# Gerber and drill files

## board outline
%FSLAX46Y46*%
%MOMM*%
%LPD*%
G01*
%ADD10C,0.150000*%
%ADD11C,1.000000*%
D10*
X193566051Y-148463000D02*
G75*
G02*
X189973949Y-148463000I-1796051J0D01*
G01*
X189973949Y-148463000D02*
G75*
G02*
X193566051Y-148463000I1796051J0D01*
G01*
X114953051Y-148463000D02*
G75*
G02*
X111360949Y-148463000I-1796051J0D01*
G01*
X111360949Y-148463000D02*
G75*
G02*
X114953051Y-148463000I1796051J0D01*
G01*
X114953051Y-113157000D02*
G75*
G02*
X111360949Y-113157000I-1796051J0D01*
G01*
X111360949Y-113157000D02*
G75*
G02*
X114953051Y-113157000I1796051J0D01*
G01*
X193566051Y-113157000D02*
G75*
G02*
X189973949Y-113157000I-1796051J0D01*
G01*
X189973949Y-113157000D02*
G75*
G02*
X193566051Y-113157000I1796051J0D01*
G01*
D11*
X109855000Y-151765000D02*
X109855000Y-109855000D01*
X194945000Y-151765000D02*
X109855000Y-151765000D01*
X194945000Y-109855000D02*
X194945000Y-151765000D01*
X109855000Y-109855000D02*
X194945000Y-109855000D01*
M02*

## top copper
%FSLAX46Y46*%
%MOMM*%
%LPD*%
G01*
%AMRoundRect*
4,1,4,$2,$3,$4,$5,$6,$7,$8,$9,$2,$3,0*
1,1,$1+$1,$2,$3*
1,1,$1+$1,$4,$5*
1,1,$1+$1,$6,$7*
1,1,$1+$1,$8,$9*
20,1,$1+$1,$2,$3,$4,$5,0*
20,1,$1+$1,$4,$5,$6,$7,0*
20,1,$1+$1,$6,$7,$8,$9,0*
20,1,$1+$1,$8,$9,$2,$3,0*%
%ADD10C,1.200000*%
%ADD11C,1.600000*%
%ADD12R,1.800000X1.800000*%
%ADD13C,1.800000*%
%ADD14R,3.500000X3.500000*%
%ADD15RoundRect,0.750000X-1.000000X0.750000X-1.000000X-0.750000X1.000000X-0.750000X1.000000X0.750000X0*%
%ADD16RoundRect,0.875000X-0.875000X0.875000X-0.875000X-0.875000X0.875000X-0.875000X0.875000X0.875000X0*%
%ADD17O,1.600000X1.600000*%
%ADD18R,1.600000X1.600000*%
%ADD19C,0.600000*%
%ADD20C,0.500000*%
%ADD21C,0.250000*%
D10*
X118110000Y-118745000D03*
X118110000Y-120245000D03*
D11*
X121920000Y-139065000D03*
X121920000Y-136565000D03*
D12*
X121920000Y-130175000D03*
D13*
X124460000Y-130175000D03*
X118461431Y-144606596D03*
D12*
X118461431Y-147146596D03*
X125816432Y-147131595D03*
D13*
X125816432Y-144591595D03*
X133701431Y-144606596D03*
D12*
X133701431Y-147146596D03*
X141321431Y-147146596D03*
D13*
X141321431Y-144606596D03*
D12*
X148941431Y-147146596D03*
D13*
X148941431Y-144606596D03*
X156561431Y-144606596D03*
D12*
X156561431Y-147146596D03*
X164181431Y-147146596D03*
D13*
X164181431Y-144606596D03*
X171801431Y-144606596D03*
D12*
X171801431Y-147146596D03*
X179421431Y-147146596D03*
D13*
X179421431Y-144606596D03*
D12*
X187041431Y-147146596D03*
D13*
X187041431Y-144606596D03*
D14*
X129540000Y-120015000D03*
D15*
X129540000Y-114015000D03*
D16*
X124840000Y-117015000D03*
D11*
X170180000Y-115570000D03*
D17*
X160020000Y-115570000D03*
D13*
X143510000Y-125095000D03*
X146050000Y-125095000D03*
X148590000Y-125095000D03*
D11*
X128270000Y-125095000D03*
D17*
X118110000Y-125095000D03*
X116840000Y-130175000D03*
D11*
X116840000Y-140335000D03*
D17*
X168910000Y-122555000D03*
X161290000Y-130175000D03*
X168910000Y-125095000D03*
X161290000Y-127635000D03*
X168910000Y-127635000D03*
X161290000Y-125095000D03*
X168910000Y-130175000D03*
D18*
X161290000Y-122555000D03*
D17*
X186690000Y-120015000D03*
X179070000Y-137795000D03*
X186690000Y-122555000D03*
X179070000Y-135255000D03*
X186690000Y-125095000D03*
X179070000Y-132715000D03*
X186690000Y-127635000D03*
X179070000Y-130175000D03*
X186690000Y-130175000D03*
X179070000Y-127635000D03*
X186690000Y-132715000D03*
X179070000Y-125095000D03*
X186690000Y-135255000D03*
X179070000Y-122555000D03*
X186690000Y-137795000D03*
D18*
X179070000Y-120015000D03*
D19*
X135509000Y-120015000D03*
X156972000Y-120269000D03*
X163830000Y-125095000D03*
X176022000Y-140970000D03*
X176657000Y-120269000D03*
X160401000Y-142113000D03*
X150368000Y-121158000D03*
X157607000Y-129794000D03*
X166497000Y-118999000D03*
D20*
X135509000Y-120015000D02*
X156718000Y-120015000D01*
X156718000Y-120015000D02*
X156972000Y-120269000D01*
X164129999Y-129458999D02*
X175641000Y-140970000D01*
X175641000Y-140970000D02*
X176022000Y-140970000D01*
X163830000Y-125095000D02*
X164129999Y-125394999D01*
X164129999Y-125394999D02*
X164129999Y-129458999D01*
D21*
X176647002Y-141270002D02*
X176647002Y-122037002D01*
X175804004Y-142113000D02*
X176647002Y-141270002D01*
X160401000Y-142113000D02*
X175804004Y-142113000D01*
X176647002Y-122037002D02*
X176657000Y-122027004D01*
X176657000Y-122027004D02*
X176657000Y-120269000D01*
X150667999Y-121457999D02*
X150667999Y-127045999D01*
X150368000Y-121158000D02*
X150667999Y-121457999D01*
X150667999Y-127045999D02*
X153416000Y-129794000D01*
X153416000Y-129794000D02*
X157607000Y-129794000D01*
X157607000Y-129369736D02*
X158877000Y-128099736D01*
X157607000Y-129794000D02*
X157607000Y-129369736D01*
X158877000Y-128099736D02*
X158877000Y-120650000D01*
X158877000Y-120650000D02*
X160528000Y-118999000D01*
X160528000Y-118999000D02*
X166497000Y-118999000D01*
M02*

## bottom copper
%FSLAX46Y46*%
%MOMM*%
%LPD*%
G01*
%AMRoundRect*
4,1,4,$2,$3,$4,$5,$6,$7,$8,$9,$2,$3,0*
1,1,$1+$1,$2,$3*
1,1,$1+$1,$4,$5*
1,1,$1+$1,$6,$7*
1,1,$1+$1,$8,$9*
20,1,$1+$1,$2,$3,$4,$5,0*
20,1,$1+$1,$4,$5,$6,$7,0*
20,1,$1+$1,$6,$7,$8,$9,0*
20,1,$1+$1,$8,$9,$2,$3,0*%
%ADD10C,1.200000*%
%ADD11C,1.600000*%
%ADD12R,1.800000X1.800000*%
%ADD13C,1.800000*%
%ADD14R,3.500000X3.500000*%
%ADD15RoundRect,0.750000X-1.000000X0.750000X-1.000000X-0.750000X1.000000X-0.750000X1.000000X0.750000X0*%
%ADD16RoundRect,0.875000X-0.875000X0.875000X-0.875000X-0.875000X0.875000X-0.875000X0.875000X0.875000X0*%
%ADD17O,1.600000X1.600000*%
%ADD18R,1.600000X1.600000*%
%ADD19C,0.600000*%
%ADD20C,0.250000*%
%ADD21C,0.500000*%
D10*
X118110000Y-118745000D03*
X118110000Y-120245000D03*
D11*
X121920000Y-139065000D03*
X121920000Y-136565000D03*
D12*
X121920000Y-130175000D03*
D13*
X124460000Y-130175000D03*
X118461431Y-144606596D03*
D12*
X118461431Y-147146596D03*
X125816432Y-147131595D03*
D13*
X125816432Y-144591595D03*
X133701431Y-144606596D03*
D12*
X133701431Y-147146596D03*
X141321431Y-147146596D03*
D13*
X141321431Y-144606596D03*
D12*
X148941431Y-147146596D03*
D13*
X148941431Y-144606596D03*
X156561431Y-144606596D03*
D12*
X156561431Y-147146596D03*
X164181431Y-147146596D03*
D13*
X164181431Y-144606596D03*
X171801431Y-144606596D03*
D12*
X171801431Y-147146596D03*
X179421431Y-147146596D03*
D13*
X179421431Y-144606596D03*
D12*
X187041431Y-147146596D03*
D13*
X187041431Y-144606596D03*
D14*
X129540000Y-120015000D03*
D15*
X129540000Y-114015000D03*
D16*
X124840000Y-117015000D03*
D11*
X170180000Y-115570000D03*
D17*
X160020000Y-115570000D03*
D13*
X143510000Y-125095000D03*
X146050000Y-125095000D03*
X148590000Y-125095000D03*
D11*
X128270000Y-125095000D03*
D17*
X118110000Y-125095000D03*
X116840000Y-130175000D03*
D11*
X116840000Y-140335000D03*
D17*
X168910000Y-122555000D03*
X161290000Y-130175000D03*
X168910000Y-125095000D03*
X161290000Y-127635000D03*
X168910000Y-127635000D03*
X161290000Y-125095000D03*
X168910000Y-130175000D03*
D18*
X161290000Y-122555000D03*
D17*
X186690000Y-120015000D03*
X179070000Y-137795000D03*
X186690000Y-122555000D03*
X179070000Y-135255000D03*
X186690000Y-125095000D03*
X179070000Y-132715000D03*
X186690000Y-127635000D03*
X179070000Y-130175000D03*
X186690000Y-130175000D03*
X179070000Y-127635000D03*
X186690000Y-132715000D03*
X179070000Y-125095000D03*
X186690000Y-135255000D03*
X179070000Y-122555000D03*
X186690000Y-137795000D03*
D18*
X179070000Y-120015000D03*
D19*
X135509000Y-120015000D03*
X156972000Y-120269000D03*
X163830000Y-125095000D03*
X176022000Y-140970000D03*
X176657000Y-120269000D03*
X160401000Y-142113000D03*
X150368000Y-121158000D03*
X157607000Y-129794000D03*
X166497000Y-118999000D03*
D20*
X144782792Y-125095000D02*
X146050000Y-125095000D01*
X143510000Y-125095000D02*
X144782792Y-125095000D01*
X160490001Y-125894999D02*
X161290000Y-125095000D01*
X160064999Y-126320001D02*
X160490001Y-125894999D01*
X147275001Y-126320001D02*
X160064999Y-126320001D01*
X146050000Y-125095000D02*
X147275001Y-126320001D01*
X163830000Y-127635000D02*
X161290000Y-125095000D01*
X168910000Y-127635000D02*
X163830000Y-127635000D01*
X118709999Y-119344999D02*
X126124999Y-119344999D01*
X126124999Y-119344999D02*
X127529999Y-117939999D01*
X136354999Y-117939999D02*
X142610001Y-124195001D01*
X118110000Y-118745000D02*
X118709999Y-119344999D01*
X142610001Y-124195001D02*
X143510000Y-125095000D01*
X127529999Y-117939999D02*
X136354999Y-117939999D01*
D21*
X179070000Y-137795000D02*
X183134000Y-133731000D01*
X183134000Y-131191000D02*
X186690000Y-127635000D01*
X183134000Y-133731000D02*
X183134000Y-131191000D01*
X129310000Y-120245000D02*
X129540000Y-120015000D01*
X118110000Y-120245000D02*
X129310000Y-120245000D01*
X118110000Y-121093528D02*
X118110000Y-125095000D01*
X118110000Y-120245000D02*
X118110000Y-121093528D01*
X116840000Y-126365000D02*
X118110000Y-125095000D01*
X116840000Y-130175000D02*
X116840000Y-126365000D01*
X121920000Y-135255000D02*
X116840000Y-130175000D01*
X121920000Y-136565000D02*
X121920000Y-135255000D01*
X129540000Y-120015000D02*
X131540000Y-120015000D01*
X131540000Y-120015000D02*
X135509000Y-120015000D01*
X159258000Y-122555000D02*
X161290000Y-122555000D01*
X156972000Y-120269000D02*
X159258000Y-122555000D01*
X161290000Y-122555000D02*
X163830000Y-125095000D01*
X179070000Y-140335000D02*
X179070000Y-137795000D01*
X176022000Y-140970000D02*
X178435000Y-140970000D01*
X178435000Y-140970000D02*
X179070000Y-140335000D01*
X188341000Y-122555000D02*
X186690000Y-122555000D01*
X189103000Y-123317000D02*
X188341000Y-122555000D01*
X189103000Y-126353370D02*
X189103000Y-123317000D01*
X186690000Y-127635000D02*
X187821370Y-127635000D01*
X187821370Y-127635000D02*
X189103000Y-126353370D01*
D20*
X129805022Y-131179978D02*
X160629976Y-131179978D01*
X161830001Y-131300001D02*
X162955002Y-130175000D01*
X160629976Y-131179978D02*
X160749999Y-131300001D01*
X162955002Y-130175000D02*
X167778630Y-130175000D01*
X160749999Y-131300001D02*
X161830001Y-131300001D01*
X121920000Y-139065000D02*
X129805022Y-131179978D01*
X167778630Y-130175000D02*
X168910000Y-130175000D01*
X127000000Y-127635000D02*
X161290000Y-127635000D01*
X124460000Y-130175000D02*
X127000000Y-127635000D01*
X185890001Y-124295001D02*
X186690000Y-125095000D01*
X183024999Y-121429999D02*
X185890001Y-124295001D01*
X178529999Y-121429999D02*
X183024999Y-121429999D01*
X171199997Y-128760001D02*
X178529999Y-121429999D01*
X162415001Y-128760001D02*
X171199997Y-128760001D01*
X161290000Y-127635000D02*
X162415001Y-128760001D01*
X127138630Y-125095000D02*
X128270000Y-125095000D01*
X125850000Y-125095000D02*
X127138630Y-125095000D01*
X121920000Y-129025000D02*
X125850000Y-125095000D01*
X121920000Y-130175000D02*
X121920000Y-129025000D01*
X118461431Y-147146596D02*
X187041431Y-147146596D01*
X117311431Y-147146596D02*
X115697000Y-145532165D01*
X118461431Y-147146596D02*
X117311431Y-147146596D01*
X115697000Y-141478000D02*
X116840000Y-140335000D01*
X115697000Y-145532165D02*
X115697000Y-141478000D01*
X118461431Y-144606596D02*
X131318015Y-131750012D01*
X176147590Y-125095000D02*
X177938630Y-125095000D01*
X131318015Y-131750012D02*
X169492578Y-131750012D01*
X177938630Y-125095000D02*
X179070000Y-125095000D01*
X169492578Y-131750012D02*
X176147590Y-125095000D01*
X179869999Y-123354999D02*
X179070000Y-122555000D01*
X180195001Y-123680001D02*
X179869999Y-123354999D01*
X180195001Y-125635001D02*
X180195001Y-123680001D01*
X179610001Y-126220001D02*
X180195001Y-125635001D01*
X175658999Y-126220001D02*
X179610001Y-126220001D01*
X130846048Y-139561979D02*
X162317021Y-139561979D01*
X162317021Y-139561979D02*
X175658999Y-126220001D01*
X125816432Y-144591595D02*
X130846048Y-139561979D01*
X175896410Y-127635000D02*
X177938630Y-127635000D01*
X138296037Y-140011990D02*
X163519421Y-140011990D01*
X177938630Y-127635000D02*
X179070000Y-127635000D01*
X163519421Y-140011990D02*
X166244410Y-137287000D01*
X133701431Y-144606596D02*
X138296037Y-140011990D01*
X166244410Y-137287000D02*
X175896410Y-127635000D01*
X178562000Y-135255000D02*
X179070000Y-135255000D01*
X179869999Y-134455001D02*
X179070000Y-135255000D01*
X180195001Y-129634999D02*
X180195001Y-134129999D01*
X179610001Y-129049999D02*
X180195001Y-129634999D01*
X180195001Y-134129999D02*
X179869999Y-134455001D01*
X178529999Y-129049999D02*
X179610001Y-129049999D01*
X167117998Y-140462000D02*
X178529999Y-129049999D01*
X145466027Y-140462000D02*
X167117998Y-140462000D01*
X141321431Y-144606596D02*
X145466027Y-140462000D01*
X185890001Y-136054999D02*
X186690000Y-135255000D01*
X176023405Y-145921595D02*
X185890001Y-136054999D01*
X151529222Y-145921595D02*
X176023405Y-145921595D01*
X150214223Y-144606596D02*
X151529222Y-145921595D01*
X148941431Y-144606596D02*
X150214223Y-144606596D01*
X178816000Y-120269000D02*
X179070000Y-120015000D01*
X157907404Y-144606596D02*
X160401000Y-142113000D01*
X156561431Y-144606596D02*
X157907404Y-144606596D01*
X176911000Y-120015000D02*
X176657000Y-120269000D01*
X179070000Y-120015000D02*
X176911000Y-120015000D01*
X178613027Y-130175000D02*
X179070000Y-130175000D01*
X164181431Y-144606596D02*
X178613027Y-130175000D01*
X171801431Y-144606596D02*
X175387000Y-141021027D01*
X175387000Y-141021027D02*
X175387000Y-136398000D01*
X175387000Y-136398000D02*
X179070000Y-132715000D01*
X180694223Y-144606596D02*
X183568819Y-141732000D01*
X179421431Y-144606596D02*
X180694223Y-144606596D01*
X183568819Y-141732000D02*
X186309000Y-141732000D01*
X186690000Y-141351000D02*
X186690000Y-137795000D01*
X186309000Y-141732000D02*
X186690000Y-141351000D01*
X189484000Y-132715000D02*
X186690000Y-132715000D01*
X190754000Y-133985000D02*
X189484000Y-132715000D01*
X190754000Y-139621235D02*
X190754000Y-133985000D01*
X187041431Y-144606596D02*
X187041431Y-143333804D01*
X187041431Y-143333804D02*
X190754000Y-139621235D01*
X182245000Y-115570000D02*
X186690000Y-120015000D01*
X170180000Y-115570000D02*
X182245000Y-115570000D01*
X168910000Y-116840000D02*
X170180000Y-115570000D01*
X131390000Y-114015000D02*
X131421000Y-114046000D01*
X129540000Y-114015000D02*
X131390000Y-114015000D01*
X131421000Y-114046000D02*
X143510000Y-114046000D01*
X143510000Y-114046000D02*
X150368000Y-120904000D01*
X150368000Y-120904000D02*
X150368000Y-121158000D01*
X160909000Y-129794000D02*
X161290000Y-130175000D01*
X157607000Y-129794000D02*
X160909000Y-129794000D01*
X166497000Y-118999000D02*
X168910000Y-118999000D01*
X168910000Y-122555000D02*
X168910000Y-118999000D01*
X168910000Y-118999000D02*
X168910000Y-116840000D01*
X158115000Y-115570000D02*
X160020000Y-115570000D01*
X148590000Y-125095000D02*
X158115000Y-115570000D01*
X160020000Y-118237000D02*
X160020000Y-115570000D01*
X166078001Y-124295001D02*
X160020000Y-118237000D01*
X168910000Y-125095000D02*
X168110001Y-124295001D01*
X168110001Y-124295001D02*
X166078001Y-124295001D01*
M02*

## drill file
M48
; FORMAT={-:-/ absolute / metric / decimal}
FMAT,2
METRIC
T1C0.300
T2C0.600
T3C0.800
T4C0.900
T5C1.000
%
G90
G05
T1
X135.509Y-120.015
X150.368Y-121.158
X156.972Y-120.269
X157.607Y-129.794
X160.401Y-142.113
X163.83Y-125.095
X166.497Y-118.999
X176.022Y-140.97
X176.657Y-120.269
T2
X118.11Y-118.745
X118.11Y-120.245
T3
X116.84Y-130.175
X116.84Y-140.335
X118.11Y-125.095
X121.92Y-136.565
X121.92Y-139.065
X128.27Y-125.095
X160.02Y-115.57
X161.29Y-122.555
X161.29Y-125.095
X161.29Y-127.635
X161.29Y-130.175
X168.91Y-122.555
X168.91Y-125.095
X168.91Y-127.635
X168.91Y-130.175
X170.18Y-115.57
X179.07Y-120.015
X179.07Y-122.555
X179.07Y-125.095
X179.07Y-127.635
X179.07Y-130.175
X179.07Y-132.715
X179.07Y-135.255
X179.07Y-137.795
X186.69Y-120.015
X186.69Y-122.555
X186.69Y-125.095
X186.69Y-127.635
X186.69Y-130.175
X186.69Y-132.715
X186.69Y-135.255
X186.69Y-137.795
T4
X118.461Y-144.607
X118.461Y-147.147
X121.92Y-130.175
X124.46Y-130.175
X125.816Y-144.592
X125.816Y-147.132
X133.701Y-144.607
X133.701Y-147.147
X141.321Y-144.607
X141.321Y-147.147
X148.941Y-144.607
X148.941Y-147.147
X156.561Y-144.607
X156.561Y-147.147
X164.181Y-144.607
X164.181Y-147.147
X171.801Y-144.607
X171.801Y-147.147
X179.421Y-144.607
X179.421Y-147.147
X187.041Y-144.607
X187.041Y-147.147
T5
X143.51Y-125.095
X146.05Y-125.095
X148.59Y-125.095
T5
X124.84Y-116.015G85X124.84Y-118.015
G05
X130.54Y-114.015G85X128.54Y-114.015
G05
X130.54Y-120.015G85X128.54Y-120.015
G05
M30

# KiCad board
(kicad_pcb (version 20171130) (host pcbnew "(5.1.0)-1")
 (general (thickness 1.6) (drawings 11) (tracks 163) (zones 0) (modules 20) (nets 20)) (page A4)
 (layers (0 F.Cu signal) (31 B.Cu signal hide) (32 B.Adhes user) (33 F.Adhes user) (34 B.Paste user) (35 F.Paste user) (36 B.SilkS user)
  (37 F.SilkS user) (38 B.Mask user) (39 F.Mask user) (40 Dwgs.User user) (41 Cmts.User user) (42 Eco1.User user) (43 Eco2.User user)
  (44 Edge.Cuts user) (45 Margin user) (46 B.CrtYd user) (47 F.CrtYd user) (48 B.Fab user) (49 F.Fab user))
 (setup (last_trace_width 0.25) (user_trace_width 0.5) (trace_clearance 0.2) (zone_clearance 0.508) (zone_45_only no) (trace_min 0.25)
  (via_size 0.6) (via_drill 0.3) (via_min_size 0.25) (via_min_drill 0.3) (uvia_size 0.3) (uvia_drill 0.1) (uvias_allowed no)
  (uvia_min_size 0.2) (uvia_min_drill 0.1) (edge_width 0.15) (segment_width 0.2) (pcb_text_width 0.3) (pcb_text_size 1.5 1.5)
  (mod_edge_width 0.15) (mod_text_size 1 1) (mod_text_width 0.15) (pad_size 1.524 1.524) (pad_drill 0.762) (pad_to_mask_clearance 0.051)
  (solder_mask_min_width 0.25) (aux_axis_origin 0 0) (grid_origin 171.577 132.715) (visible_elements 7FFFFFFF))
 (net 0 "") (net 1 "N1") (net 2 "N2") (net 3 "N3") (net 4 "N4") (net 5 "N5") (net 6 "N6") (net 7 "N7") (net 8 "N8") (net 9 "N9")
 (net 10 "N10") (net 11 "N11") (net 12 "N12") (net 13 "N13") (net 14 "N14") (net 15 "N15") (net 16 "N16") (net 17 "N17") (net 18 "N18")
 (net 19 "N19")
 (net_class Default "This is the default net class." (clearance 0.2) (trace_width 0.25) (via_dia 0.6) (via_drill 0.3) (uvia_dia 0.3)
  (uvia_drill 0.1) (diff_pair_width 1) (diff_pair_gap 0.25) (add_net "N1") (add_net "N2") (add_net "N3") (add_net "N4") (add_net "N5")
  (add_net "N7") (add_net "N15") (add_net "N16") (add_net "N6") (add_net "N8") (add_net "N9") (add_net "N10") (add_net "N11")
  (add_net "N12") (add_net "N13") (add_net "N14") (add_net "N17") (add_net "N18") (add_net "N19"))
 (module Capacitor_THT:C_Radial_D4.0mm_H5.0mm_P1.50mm (layer F.Cu) (at 118.11 118.745 270)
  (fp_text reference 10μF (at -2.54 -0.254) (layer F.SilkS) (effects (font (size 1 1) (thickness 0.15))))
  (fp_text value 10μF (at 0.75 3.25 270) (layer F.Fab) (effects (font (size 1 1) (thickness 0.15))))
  (pad 1 thru_hole circle (at 0 0 270) (size 1.2 1.2) (drill 0.6) (layers *.Cu *.Mask) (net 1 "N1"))
  (pad 2 thru_hole circle (at 1.5 0 270) (size 1.2 1.2) (drill 0.6) (layers *.Cu *.Mask) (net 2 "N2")))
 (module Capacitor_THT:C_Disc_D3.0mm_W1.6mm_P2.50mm (layer F.Cu) (at 121.92 139.065 90)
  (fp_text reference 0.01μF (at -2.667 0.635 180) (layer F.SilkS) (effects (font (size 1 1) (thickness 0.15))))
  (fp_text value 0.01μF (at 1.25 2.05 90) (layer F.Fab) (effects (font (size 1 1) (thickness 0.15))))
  (pad 1 thru_hole circle (at 0 0 90) (size 1.6 1.6) (drill 0.8) (layers *.Cu *.Mask) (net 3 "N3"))
  (pad 2 thru_hole circle (at 2.5 0 90) (size 1.6 1.6) (drill 0.8) (layers *.Cu *.Mask) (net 2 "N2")))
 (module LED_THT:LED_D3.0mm (layer F.Cu) (at 121.92 130.175)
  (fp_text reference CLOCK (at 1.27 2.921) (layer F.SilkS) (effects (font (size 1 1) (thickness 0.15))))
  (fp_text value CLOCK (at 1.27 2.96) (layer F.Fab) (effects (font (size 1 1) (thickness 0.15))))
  (pad 1 thru_hole rect (at 0 0) (size 1.8 1.8) (drill 0.9) (layers *.Cu *.Mask) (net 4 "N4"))
  (pad 2 thru_hole circle (at 2.54 0) (size 1.8 1.8) (drill 0.9) (layers *.Cu *.Mask) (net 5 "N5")))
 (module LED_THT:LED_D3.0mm (layer F.Cu) (at 118.461431 147.146596 90)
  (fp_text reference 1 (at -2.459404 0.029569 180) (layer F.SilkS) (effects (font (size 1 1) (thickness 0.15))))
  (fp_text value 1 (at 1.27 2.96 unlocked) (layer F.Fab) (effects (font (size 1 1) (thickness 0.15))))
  (pad 2 thru_hole circle (at 2.54 0 90) (size 1.8 1.8) (drill 0.9) (layers *.Cu *.Mask) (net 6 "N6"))
  (pad 1 thru_hole rect (at 0 0 90) (size 1.8 1.8) (drill 0.9) (layers *.Cu *.Mask) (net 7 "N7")))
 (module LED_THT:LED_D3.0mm (layer F.Cu) (at 125.816432 147.131595 90)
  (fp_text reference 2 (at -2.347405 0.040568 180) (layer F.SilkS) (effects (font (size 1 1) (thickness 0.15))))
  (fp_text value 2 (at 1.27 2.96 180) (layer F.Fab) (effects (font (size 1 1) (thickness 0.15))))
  (pad 1 thru_hole rect (at 0 0 90) (size 1.8 1.8) (drill 0.9) (layers *.Cu *.Mask) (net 7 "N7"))
  (pad 2 thru_hole circle (at 2.54 0 90) (size 1.8 1.8) (drill 0.9) (layers *.Cu *.Mask) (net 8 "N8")))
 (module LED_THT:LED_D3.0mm (layer F.Cu) (at 133.701431 147.146596 90)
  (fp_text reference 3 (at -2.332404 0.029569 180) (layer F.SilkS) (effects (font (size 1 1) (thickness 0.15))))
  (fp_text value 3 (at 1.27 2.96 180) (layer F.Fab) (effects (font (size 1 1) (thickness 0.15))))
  (pad 2 thru_hole circle (at 2.54 0 90) (size 1.8 1.8) (drill 0.9) (layers *.Cu *.Mask) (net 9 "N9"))
  (pad 1 thru_hole rect (at 0 0 90) (size 1.8 1.8) (drill 0.9) (layers *.Cu *.Mask) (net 7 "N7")))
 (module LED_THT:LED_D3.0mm (layer F.Cu) (at 141.321431 147.146596 90)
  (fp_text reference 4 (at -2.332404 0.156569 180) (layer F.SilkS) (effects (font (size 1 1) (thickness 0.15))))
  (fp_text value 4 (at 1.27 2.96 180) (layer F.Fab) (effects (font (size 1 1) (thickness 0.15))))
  (pad 1 thru_hole rect (at 0 0 90) (size 1.8 1.8) (drill 0.9) (layers *.Cu *.Mask) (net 7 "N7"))
  (pad 2 thru_hole circle (at 2.54 0 90) (size 1.8 1.8) (drill 0.9) (layers *.Cu *.Mask) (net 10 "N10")))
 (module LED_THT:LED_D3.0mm (layer F.Cu) (at 148.941431 147.146596 90)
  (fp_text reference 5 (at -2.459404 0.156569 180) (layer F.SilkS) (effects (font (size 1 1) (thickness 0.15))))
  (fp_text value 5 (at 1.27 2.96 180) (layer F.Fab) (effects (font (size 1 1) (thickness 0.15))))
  (pad 1 thru_hole rect (at 0 0 90) (size 1.8 1.8) (drill 0.9) (layers *.Cu *.Mask) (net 7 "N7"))
  (pad 2 thru_hole circle (at 2.54 0 90) (size 1.8 1.8) (drill 0.9) (layers *.Cu *.Mask) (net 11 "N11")))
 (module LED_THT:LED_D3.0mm (layer F.Cu) (at 156.561431 147.146596 90)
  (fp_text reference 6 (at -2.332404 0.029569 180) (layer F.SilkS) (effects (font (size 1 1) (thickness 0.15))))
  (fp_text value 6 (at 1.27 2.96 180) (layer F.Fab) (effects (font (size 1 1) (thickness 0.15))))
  (pad 2 thru_hole circle (at 2.54 0 90) (size 1.8 1.8) (drill 0.9) (layers *.Cu *.Mask) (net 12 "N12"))
  (pad 1 thru_hole rect (at 0 0 90) (size 1.8 1.8) (drill 0.9) (layers *.Cu *.Mask) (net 7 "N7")))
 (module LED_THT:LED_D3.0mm (layer F.Cu) (at 164.181431 147.146596 90)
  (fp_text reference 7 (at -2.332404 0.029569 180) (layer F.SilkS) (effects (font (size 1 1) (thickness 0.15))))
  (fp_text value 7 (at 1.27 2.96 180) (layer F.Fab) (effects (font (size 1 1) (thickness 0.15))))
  (pad 1 thru_hole rect (at 0 0 90) (size 1.8 1.8) (drill 0.9) (layers *.Cu *.Mask) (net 7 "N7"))
  (pad 2 thru_hole circle (at 2.54 0 90) (size 1.8 1.8) (drill 0.9) (layers *.Cu *.Mask) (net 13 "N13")))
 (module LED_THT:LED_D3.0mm (layer F.Cu) (at 171.801431 147.146596 90)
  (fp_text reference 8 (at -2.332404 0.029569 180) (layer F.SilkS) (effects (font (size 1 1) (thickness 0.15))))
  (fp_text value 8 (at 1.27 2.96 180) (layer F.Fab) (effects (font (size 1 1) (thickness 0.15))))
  (pad 2 thru_hole circle (at 2.54 0 90) (size 1.8 1.8) (drill 0.9) (layers *.Cu *.Mask) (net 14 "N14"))
  (pad 1 thru_hole rect (at 0 0 90) (size 1.8 1.8) (drill 0.9) (layers *.Cu *.Mask) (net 7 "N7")))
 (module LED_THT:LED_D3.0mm (layer F.Cu) (at 179.421431 147.146596 90)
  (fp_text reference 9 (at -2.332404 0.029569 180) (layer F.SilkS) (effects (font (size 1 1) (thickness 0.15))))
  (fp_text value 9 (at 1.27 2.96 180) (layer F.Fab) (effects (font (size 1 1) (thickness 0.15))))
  (pad 1 thru_hole rect (at 0 0 90) (size 1.8 1.8) (drill 0.9) (layers *.Cu *.Mask) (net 7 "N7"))
  (pad 2 thru_hole circle (at 2.54 0 90) (size 1.8 1.8) (drill 0.9) (layers *.Cu *.Mask) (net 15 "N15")))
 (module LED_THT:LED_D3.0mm (layer F.Cu) (at 187.041431 147.146596 90)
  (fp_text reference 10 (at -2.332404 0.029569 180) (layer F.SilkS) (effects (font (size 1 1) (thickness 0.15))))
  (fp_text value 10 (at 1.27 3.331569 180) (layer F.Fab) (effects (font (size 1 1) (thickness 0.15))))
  (pad 1 thru_hole rect (at 0 0 90) (size 1.8 1.8) (drill 0.9) (layers *.Cu *.Mask) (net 7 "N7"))
  (pad 2 thru_hole circle (at 2.54 0 90) (size 1.8 1.8) (drill 0.9) (layers *.Cu *.Mask) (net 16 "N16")))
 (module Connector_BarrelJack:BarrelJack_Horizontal (layer F.Cu) (at 129.54 120.015 270)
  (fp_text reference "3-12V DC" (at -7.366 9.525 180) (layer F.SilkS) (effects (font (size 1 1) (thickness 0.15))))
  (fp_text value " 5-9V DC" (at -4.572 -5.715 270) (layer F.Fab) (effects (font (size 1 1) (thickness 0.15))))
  (pad 1 thru_hole rect (at 0 0 270) (size 3.5 3.5) (drill oval 1 3) (layers *.Cu *.Mask) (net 2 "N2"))
  (pad 2 thru_hole roundrect (at -6 0 270) (size 3 3.5) (drill oval 1 3) (layers *.Cu *.Mask) (roundrect_rratio 0.25) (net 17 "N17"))
  (pad 3 thru_hole roundrect (at -3 4.7 270) (size 3.5 3.5) (drill oval 3 1) (layers *.Cu *.Mask) (roundrect_rratio 0.25)))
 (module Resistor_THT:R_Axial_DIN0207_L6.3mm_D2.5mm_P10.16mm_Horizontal (layer F.Cu) (at 170.18 115.57 180)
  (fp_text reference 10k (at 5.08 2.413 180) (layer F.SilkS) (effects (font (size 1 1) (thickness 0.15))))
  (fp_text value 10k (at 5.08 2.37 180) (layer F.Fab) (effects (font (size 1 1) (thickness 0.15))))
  (pad 1 thru_hole circle (at 0 0 180) (size 1.6 1.6) (drill 0.8) (layers *.Cu *.Mask) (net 17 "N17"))
  (pad 2 thru_hole oval (at 10.16 0 180) (size 1.6 1.6) (drill 0.8) (layers *.Cu *.Mask) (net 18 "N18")))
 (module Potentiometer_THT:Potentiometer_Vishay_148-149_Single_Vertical (layer F.Cu) (at 148.59 125.095 90)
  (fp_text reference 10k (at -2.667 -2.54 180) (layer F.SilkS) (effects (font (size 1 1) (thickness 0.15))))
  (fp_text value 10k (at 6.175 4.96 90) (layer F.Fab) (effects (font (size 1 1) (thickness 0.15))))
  (pad 3 thru_hole circle (at 0 -5.08 90) (size 1.8 1.8) (drill 1) (layers *.Cu *.Mask) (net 1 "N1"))
  (pad 2 thru_hole circle (at 0 -2.54 90) (size 1.8 1.8) (drill 1) (layers *.Cu *.Mask) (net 1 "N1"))
  (pad 1 thru_hole circle (at 0 0 90) (size 1.8 1.8) (drill 1) (layers *.Cu *.Mask) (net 18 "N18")))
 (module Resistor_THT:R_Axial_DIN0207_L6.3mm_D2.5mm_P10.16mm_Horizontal (layer F.Cu) (at 128.27 125.095 180)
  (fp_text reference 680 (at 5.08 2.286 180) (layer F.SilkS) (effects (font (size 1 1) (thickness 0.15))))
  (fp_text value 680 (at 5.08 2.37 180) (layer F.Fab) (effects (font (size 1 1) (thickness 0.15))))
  (pad 1 thru_hole circle (at 0 0 180) (size 1.6 1.6) (drill 0.8) (layers *.Cu *.Mask) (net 4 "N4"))
  (pad 2 thru_hole oval (at 10.16 0 180) (size 1.6 1.6) (drill 0.8) (layers *.Cu *.Mask) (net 2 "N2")))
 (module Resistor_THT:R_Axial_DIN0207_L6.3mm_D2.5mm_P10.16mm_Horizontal (layer F.Cu) (at 116.84 140.335 90)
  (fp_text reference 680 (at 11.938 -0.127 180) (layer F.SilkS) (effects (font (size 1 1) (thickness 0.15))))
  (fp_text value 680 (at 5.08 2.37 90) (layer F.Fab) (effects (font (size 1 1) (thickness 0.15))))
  (pad 2 thru_hole oval (at 10.16 0 90) (size 1.6 1.6) (drill 0.8) (layers *.Cu *.Mask) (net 2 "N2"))
  (pad 1 thru_hole circle (at 0 0 90) (size 1.6 1.6) (drill 0.8) (layers *.Cu *.Mask) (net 7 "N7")))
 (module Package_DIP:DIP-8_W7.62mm (layer F.Cu) (at 161.29 122.555)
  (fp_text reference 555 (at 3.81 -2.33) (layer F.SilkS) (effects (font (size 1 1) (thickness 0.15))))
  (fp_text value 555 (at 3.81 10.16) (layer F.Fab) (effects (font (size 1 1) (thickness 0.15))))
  (pad 8 thru_hole oval (at 7.62 0) (size 1.6 1.6) (drill 0.8) (layers *.Cu *.Mask) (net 17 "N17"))
  (pad 4 thru_hole oval (at 0 7.62) (size 1.6 1.6) (drill 0.8) (layers *.Cu *.Mask) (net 17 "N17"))
  (pad 7 thru_hole oval (at 7.62 2.54) (size 1.6 1.6) (drill 0.8) (layers *.Cu *.Mask) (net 18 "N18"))
  (pad 3 thru_hole oval (at 0 5.08) (size 1.6 1.6) (drill 0.8) (layers *.Cu *.Mask) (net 5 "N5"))
  (pad 6 thru_hole oval (at 7.62 5.08) (size 1.6 1.6) (drill 0.8) (layers *.Cu *.Mask) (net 1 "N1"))
  (pad 2 thru_hole oval (at 0 2.54) (size 1.6 1.6) (drill 0.8) (layers *.Cu *.Mask) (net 1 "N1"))
  (pad 5 thru_hole oval (at 7.62 7.62) (size 1.6 1.6) (drill 0.8) (layers *.Cu *.Mask) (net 3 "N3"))
  (pad 1 thru_hole rect (at 0 0) (size 1.6 1.6) (drill 0.8) (layers *.Cu *.Mask) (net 2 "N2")))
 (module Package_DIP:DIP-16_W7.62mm (layer F.Cu) (at 179.07 120.015)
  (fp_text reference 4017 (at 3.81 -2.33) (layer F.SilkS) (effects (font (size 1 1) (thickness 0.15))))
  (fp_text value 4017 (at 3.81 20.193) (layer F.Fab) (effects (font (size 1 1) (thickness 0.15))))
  (pad 16 thru_hole oval (at 7.62 0) (size 1.6 1.6) (drill 0.8) (layers *.Cu *.Mask) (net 17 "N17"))
  (pad 8 thru_hole oval (at 0 17.78) (size 1.6 1.6) (drill 0.8) (layers *.Cu *.Mask) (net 2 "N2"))
  (pad 15 thru_hole oval (at 7.62 2.54) (size 1.6 1.6) (drill 0.8) (layers *.Cu *.Mask) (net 2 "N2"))
  (pad 7 thru_hole oval (at 0 15.24) (size 1.6 1.6) (drill 0.8) (layers *.Cu *.Mask) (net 10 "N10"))
  (pad 14 thru_hole oval (at 7.62 5.08) (size 1.6 1.6) (drill 0.8) (layers *.Cu *.Mask) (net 5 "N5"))
  (pad 6 thru_hole oval (at 0 12.7) (size 1.6 1.6) (drill 0.8) (layers *.Cu *.Mask) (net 14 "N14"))
  (pad 13 thru_hole oval (at 7.62 7.62) (size 1.6 1.6) (drill 0.8) (layers *.Cu *.Mask) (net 2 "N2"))
  (pad 5 thru_hole oval (at 0 10.16) (size 1.6 1.6) (drill 0.8) (layers *.Cu *.Mask) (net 13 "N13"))
  (pad 12 thru_hole oval (at 7.62 10.16) (size 1.6 1.6) (drill 0.8) (layers *.Cu *.Mask) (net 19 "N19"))
  (pad 4 thru_hole oval (at 0 7.62) (size 1.6 1.6) (drill 0.8) (layers *.Cu *.Mask) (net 9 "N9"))
  (pad 11 thru_hole oval (at 7.62 12.7) (size 1.6 1.6) (drill 0.8) (layers *.Cu *.Mask) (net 16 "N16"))
  (pad 3 thru_hole oval (at 0 5.08) (size 1.6 1.6) (drill 0.8) (layers *.Cu *.Mask) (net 6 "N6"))
  (pad 10 thru_hole oval (at 7.62 15.24) (size 1.6 1.6) (drill 0.8) (layers *.Cu *.Mask) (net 11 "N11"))
  (pad 2 thru_hole oval (at 0 2.54) (size 1.6 1.6) (drill 0.8) (layers *.Cu *.Mask) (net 8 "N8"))
  (pad 9 thru_hole oval (at 7.62 17.78) (size 1.6 1.6) (drill 0.8) (layers *.Cu *.Mask) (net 15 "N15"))
  (pad 1 thru_hole rect (at 0 0) (size 1.6 1.6) (drill 0.8) (layers *.Cu *.Mask) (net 12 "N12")))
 (gr_circle (center 191.77 148.463) (end 193.566051 148.463) (layer Edge.Cuts) (width 0.15))
 (gr_circle (center 113.157 148.463) (end 114.953051 148.463) (layer Edge.Cuts) (width 0.15))
 (gr_circle (center 113.157 113.157) (end 114.953051 113.157) (layer Edge.Cuts) (width 0.15))
 (gr_circle (center 191.77 113.157) (end 193.566051 113.157) (layer Edge.Cuts) (width 0.15))
 (gr_line (start 109.855 151.765) (end 109.855 109.855) (layer Edge.Cuts) (width 1))
 (gr_line (start 194.945 151.765) (end 109.855 151.765) (layer Edge.Cuts) (width 1))
 (gr_line (start 194.945 109.855) (end 194.945 151.765) (layer Edge.Cuts) (width 1))
 (gr_line (start 109.855 109.855) (end 194.945 109.855) (layer Edge.Cuts) (width 1))
 (segment (start 144.782792 125.095) (end 146.05 125.095) (width 0.25) (layer B.Cu) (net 1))
 (segment (start 143.51 125.095) (end 144.782792 125.095) (width 0.25) (layer B.Cu) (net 1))
 (segment (start 160.490001 125.894999) (end 161.29 125.095) (width 0.25) (layer B.Cu) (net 1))
 (segment (start 160.064999 126.320001) (end 160.490001 125.894999) (width 0.25) (layer B.Cu) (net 1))
 (segment (start 147.275001 126.320001) (end 160.064999 126.320001) (width 0.25) (layer B.Cu) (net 1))
 (segment (start 146.05 125.095) (end 147.275001 126.320001) (width 0.25) (layer B.Cu) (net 1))
 (segment (start 163.83 127.635) (end 161.29 125.095) (width 0.25) (layer B.Cu) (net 1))
 (segment (start 168.91 127.635) (end 163.83 127.635) (width 0.25) (layer B.Cu) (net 1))
 (segment (start 118.709999 119.344999) (end 126.124999 119.344999) (width 0.25) (layer B.Cu) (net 1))
 (segment (start 126.124999 119.344999) (end 127.529999 117.939999) (width 0.25) (layer B.Cu) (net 1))
 (segment (start 136.354999 117.939999) (end 142.610001 124.195001) (width 0.25) (layer B.Cu) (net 1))
 (segment (start 118.11 118.745) (end 118.709999 119.344999) (width 0.25) (layer B.Cu) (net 1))
 (segment (start 142.610001 124.195001) (end 143.51 125.095) (width 0.25) (layer B.Cu) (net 1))
 (segment (start 127.529999 117.939999) (end 136.354999 117.939999) (width 0.25) (layer B.Cu) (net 1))
 (segment (start 179.07 137.795) (end 183.134 133.731) (width 0.5) (layer B.Cu) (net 2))
 (segment (start 183.134 131.191) (end 186.69 127.635) (width 0.5) (layer B.Cu) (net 2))
 (segment (start 183.134 133.731) (end 183.134 131.191) (width 0.5) (layer B.Cu) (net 2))
 (segment (start 129.31 120.245) (end 129.54 120.015) (width 0.5) (layer B.Cu) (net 2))
 (segment (start 118.11 120.245) (end 129.31 120.245) (width 0.5) (layer B.Cu) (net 2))
 (segment (start 118.11 121.093528) (end 118.11 125.095) (width 0.5) (layer B.Cu) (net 2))
 (segment (start 118.11 120.245) (end 118.11 121.093528) (width 0.5) (layer B.Cu) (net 2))
 (segment (start 116.84 126.365) (end 118.11 125.095) (width 0.5) (layer B.Cu) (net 2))
 (segment (start 116.84 130.175) (end 116.84 126.365) (width 0.5) (layer B.Cu) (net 2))
 (segment (start 121.92 135.255) (end 116.84 130.175) (width 0.5) (layer B.Cu) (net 2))
 (segment (start 121.92 136.565) (end 121.92 135.255) (width 0.5) (layer B.Cu) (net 2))
 (segment (start 129.54 120.015) (end 131.54 120.015) (width 0.5) (layer B.Cu) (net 2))
 (via (at 135.509 120.015) (size 0.6) (drill 0.3) (layers F.Cu B.Cu) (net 2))
 (segment (start 131.54 120.015) (end 135.509 120.015) (width 0.5) (layer B.Cu) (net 2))
 (via (at 156.972 120.269) (size 0.6) (drill 0.3) (layers F.Cu B.Cu) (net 2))
 (segment (start 135.509 120.015) (end 156.718 120.015) (width 0.5) (layer F.Cu) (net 2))
 (segment (start 156.718 120.015) (end 156.972 120.269) (width 0.5) (layer F.Cu) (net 2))
 (segment (start 159.258 122.555) (end 161.29 122.555) (width 0.5) (layer B.Cu) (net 2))
 (segment (start 156.972 120.269) (end 159.258 122.555) (width 0.5) (layer B.Cu) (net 2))
 (via (at 163.83 125.095) (size 0.6) (drill 0.3) (layers F.Cu B.Cu) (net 2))
 (segment (start 164.129999 129.458999) (end 175.641 140.97) (width 0.5) (layer F.Cu) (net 2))
 (segment (start 175.641 140.97) (end 176.022 140.97) (width 0.5) (layer F.Cu) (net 2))
 (via (at 176.022 140.97) (size 0.6) (drill 0.3) (layers F.Cu B.Cu) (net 2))
 (segment (start 163.83 125.095) (end 164.129999 125.394999) (width 0.5) (layer F.Cu) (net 2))
 (segment (start 164.129999 125.394999) (end 164.129999 129.458999) (width 0.5) (layer F.Cu) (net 2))
 (segment (start 161.29 122.555) (end 163.83 125.095) (width 0.5) (layer B.Cu) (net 2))
 (segment (start 179.07 140.335) (end 179.07 137.795) (width 0.5) (layer B.Cu) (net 2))
 (segment (start 176.022 140.97) (end 178.435 140.97) (width 0.5) (layer B.Cu) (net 2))
 (segment (start 178.435 140.97) (end 179.07 140.335) (width 0.5) (layer B.Cu) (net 2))
 (segment (start 188.341 122.555) (end 186.69 122.555) (width 0.5) (layer B.Cu) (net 2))
 (segment (start 189.103 123.317) (end 188.341 122.555) (width 0.5) (layer B.Cu) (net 2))
 (segment (start 189.103 126.35337) (end 189.103 123.317) (width 0.5) (layer B.Cu) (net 2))
 (segment (start 186.69 127.635) (end 187.82137 127.635) (width 0.5) (layer B.Cu) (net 2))
 (segment (start 187.82137 127.635) (end 189.103 126.35337) (width 0.5) (layer B.Cu) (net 2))
 (segment (start 129.805022 131.179978) (end 160.629976 131.179978) (width 0.25) (layer B.Cu) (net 3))
 (segment (start 161.830001 131.300001) (end 162.955002 130.175) (width 0.25) (layer B.Cu) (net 3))
 (segment (start 160.629976 131.179978) (end 160.749999 131.300001) (width 0.25) (layer B.Cu) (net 3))
 (segment (start 162.955002 130.175) (end 167.77863 130.175) (width 0.25) (layer B.Cu) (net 3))
 (segment (start 160.749999 131.300001) (end 161.830001 131.300001) (width 0.25) (layer B.Cu) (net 3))
 (segment (start 121.92 139.065) (end 129.805022 131.179978) (width 0.25) (layer B.Cu) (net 3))
 (segment (start 167.77863 130.175) (end 168.91 130.175) (width 0.25) (layer B.Cu) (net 3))
 (segment (start 127 127.635) (end 161.29 127.635) (width 0.25) (layer B.Cu) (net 5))
 (segment (start 124.46 130.175) (end 127 127.635) (width 0.25) (layer B.Cu) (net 5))
 (segment (start 185.890001 124.295001) (end 186.69 125.095) (width 0.25) (layer B.Cu) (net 5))
 (segment (start 183.024999 121.429999) (end 185.890001 124.295001) (width 0.25) (layer B.Cu) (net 5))
 (segment (start 178.529999 121.429999) (end 183.024999 121.429999) (width 0.25) (layer B.Cu) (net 5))
 (segment (start 171.199997 128.760001) (end 178.529999 121.429999) (width 0.25) (layer B.Cu) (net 5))
 (segment (start 162.415001 128.760001) (end 171.199997 128.760001) (width 0.25) (layer B.Cu) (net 5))
 (segment (start 161.29 127.635) (end 162.415001 128.760001) (width 0.25) (layer B.Cu) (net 5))
 (segment (start 127.13863 125.095) (end 128.27 125.095) (width 0.25) (layer B.Cu) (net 4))
 (segment (start 125.85 125.095) (end 127.13863 125.095) (width 0.25) (layer B.Cu) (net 4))
 (segment (start 121.92 129.025) (end 125.85 125.095) (width 0.25) (layer B.Cu) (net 4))
 (segment (start 121.92 130.175) (end 121.92 129.025) (width 0.25) (layer B.Cu) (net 4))
 (segment (start 118.461431 147.146596) (end 187.041431 147.146596) (width 0.25) (layer B.Cu) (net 7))
 (segment (start 117.311431 147.146596) (end 115.697 145.532165) (width 0.25) (layer B.Cu) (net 7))
 (segment (start 118.461431 147.146596) (end 117.311431 147.146596) (width 0.25) (layer B.Cu) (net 7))
 (segment (start 115.697 141.478) (end 116.84 140.335) (width 0.25) (layer B.Cu) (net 7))
 (segment (start 115.697 145.532165) (end 115.697 141.478) (width 0.25) (layer B.Cu) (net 7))
 (segment (start 118.461431 144.606596) (end 131.318015 131.750012) (width 0.25) (layer B.Cu) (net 6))
 (segment (start 176.14759 125.095) (end 177.93863 125.095) (width 0.25) (layer B.Cu) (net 6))
 (segment (start 131.318015 131.750012) (end 169.492578 131.750012) (width 0.25) (layer B.Cu) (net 6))
 (segment (start 177.93863 125.095) (end 179.07 125.095) (width 0.25) (layer B.Cu) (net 6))
 (segment (start 169.492578 131.750012) (end 176.14759 125.095) (width 0.25) (layer B.Cu) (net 6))
 (segment (start 179.869999 123.354999) (end 179.07 122.555) (width 0.25) (layer B.Cu) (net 8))
 (segment (start 180.195001 123.680001) (end 179.869999 123.354999) (width 0.25) (layer B.Cu) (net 8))
 (segment (start 180.195001 125.635001) (end 180.195001 123.680001) (width 0.25) (layer B.Cu) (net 8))
 (segment (start 179.610001 126.220001) (end 180.195001 125.635001) (width 0.25) (layer B.Cu) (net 8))
 (segment (start 175.658999 126.220001) (end 179.610001 126.220001) (width 0.25) (layer B.Cu) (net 8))
 (segment (start 130.846048 139.561979) (end 162.317021 139.561979) (width 0.25) (layer B.Cu) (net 8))
 (segment (start 162.317021 139.561979) (end 175.658999 126.220001) (width 0.25) (layer B.Cu) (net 8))
 (segment (start 125.816432 144.591595) (end 130.846048 139.561979) (width 0.25) (layer B.Cu) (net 8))
 (segment (start 175.89641 127.635) (end 177.93863 127.635) (width 0.25) (layer B.Cu) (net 9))
 (segment (start 138.296037 140.01199) (end 163.519421 140.01199) (width 0.25) (layer B.Cu) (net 9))
 (segment (start 177.93863 127.635) (end 179.07 127.635) (width 0.25) (layer B.Cu) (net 9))
 (segment (start 163.519421 140.01199) (end 166.24441 137.287) (width 0.25) (layer B.Cu) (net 9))
 (segment (start 133.701431 144.606596) (end 138.296037 140.01199) (width 0.25) (layer B.Cu) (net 9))
 (segment (start 166.24441 137.287) (end 175.89641 127.635) (width 0.25) (layer B.Cu) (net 9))
 (segment (start 178.562 135.255) (end 179.07 135.255) (width 0.25) (layer B.Cu) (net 10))
 (segment (start 179.869999 134.455001) (end 179.07 135.255) (width 0.25) (layer B.Cu) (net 10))
 (segment (start 180.195001 129.634999) (end 180.195001 134.129999) (width 0.25) (layer B.Cu) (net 10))
 (segment (start 179.610001 129.049999) (end 180.195001 129.634999) (width 0.25) (layer B.Cu) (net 10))
 (segment (start 180.195001 134.129999) (end 179.869999 134.455001) (width 0.25) (layer B.Cu) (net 10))
 (segment (start 178.529999 129.049999) (end 179.610001 129.049999) (width 0.25) (layer B.Cu) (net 10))
 (segment (start 167.117998 140.462) (end 178.529999 129.049999) (width 0.25) (layer B.Cu) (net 10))
 (segment (start 145.466027 140.462) (end 167.117998 140.462) (width 0.25) (layer B.Cu) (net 10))
 (segment (start 141.321431 144.606596) (end 145.466027 140.462) (width 0.25) (layer B.Cu) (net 10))
 (segment (start 185.890001 136.054999) (end 186.69 135.255) (width 0.25) (layer B.Cu) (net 11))
 (segment (start 176.023405 145.921595) (end 185.890001 136.054999) (width 0.25) (layer B.Cu) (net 11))
 (segment (start 151.529222 145.921595) (end 176.023405 145.921595) (width 0.25) (layer B.Cu) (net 11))
 (segment (start 150.214223 144.606596) (end 151.529222 145.921595) (width 0.25) (layer B.Cu) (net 11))
 (segment (start 148.941431 144.606596) (end 150.214223 144.606596) (width 0.25) (layer B.Cu) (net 11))
 (segment (start 178.816 120.269) (end 179.07 120.015) (width 0.25) (layer B.Cu) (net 12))
 (segment (start 176.647002 141.270002) (end 176.647002 122.037002) (width 0.25) (layer F.Cu) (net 12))
 (segment (start 175.804004 142.113) (end 176.647002 141.270002) (width 0.25) (layer F.Cu) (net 12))
 (segment (start 160.401 142.113) (end 175.804004 142.113) (width 0.25) (layer F.Cu) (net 12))
 (segment (start 176.647002 122.037002) (end 176.657 122.027004) (width 0.25) (layer F.Cu) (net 12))
 (segment (start 176.657 122.027004) (end 176.657 120.269) (width 0.25) (layer F.Cu) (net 12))
 (via (at 176.657 120.269) (size 0.6) (drill 0.3) (layers F.Cu B.Cu) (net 12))
 (via (at 160.401 142.113) (size 0.6) (drill 0.3) (layers F.Cu B.Cu) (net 12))
 (segment (start 157.907404 144.606596) (end 160.401 142.113) (width 0.25) (layer B.Cu) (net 12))
 (segment (start 156.561431 144.606596) (end 157.907404 144.606596) (width 0.25) (layer B.Cu) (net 12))
 (segment (start 176.911 120.015) (end 176.657 120.269) (width 0.25) (layer B.Cu) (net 12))
 (segment (start 179.07 120.015) (end 176.911 120.015) (width 0.25) (layer B.Cu) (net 12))
 (segment (start 178.613027 130.175) (end 179.07 130.175) (width 0.25) (layer B.Cu) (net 13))
 (segment (start 164.181431 144.606596) (end 178.613027 130.175) (width 0.25) (layer B.Cu) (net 13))
 (segment (start 171.801431 144.606596) (end 175.387 141.021027) (width 0.25) (layer B.Cu) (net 14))
 (segment (start 175.387 141.021027) (end 175.387 136.398) (width 0.25) (layer B.Cu) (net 14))
 (segment (start 175.387 136.398) (end 179.07 132.715) (width 0.25) (layer B.Cu) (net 14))
 (segment (start 180.694223 144.606596) (end 183.568819 141.732) (width 0.25) (layer B.Cu) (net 15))
 (segment (start 179.421431 144.606596) (end 180.694223 144.606596) (width 0.25) (layer B.Cu) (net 15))
 (segment (start 183.568819 141.732) (end 186.309 141.732) (width 0.25) (layer B.Cu) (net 15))
 (segment (start 186.69 141.351) (end 186.69 137.795) (width 0.25) (layer B.Cu) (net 15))
 (segment (start 186.309 141.732) (end 186.69 141.351) (width 0.25) (layer B.Cu) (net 15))
 (segment (start 189.484 132.715) (end 186.69 132.715) (width 0.25) (layer B.Cu) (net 16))
 (segment (start 190.754 133.985) (end 189.484 132.715) (width 0.25) (layer B.Cu) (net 16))
 (segment (start 190.754 139.621235) (end 190.754 133.985) (width 0.25) (layer B.Cu) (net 16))
 (segment (start 187.041431 144.606596) (end 187.041431 143.333804) (width 0.25) (layer B.Cu) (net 16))
 (segment (start 187.041431 143.333804) (end 190.754 139.621235) (width 0.25) (layer B.Cu) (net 16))
 (segment (start 182.245 115.57) (end 186.69 120.015) (width 0.25) (layer B.Cu) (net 17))
 (segment (start 170.18 115.57) (end 182.245 115.57) (width 0.25) (layer B.Cu) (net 17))
 (segment (start 168.91 116.84) (end 170.18 115.57) (width 0.25) (layer B.Cu) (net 17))
 (segment (start 131.39 114.015) (end 131.421 114.046) (width 0.25) (layer B.Cu) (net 17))
 (segment (start 129.54 114.015) (end 131.39 114.015) (width 0.25) (layer B.Cu) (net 17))
 (segment (start 131.421 114.046) (end 143.51 114.046) (width 0.25) (layer B.Cu) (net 17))
 (via (at 150.368 121.158) (size 0.6) (drill 0.3) (layers F.Cu B.Cu) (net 17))
 (segment (start 143.51 114.046) (end 150.368 120.904) (width 0.25) (layer B.Cu) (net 17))
 (segment (start 150.368 120.904) (end 150.368 121.158) (width 0.25) (layer B.Cu) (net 17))
 (segment (start 150.667999 121.457999) (end 150.667999 127.045999) (width 0.25) (layer F.Cu) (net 17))
 (segment (start 150.368 121.158) (end 150.667999 121.457999) (width 0.25) (layer F.Cu) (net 17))
 (segment (start 150.667999 127.045999) (end 153.416 129.794) (width 0.25) (layer F.Cu) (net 17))
 (via (at 157.607 129.794) (size 0.6) (drill 0.3) (layers F.Cu B.Cu) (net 17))
 (segment (start 153.416 129.794) (end 157.607 129.794) (width 0.25) (layer F.Cu) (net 17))
 (segment (start 160.909 129.794) (end 161.29 130.175) (width 0.25) (layer B.Cu) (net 17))
 (segment (start 157.607 129.794) (end 160.909 129.794) (width 0.25) (layer B.Cu) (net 17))
 (segment (start 157.607 129.369736) (end 158.877 128.099736) (width 0.25) (layer F.Cu) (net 17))
 (segment (start 157.607 129.794) (end 157.607 129.369736) (width 0.25) (layer F.Cu) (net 17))
 (segment (start 158.877 128.099736) (end 158.877 120.65) (width 0.25) (layer F.Cu) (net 17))
 (segment (start 158.877 120.65) (end 160.528 118.999) (width 0.25) (layer F.Cu) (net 17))
 (segment (start 160.528 118.999) (end 166.497 118.999) (width 0.25) (layer F.Cu) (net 17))
 (via (at 166.497 118.999) (size 0.6) (drill 0.3) (layers F.Cu B.Cu) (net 17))
 (segment (start 166.497 118.999) (end 168.91 118.999) (width 0.25) (layer B.Cu) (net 17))
 (segment (start 168.91 122.555) (end 168.91 118.999) (width 0.25) (layer B.Cu) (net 17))
 (segment (start 168.91 118.999) (end 168.91 116.84) (width 0.25) (layer B.Cu) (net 17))
 (segment (start 158.115 115.57) (end 160.02 115.57) (width 0.25) (layer B.Cu) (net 18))
 (segment (start 148.59 125.095) (end 158.115 115.57) (width 0.25) (layer B.Cu) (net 18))
 (segment (start 160.02 118.237) (end 160.02 115.57) (width 0.25) (layer B.Cu) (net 18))
 (segment (start 166.078001 124.295001) (end 160.02 118.237) (width 0.25) (layer B.Cu) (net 18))
 (segment (start 168.91 125.095) (end 168.110001 124.295001) (width 0.25) (layer B.Cu) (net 18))
 (segment (start 168.110001 124.295001) (end 166.078001 124.295001) (width 0.25) (layer B.Cu) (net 18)))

